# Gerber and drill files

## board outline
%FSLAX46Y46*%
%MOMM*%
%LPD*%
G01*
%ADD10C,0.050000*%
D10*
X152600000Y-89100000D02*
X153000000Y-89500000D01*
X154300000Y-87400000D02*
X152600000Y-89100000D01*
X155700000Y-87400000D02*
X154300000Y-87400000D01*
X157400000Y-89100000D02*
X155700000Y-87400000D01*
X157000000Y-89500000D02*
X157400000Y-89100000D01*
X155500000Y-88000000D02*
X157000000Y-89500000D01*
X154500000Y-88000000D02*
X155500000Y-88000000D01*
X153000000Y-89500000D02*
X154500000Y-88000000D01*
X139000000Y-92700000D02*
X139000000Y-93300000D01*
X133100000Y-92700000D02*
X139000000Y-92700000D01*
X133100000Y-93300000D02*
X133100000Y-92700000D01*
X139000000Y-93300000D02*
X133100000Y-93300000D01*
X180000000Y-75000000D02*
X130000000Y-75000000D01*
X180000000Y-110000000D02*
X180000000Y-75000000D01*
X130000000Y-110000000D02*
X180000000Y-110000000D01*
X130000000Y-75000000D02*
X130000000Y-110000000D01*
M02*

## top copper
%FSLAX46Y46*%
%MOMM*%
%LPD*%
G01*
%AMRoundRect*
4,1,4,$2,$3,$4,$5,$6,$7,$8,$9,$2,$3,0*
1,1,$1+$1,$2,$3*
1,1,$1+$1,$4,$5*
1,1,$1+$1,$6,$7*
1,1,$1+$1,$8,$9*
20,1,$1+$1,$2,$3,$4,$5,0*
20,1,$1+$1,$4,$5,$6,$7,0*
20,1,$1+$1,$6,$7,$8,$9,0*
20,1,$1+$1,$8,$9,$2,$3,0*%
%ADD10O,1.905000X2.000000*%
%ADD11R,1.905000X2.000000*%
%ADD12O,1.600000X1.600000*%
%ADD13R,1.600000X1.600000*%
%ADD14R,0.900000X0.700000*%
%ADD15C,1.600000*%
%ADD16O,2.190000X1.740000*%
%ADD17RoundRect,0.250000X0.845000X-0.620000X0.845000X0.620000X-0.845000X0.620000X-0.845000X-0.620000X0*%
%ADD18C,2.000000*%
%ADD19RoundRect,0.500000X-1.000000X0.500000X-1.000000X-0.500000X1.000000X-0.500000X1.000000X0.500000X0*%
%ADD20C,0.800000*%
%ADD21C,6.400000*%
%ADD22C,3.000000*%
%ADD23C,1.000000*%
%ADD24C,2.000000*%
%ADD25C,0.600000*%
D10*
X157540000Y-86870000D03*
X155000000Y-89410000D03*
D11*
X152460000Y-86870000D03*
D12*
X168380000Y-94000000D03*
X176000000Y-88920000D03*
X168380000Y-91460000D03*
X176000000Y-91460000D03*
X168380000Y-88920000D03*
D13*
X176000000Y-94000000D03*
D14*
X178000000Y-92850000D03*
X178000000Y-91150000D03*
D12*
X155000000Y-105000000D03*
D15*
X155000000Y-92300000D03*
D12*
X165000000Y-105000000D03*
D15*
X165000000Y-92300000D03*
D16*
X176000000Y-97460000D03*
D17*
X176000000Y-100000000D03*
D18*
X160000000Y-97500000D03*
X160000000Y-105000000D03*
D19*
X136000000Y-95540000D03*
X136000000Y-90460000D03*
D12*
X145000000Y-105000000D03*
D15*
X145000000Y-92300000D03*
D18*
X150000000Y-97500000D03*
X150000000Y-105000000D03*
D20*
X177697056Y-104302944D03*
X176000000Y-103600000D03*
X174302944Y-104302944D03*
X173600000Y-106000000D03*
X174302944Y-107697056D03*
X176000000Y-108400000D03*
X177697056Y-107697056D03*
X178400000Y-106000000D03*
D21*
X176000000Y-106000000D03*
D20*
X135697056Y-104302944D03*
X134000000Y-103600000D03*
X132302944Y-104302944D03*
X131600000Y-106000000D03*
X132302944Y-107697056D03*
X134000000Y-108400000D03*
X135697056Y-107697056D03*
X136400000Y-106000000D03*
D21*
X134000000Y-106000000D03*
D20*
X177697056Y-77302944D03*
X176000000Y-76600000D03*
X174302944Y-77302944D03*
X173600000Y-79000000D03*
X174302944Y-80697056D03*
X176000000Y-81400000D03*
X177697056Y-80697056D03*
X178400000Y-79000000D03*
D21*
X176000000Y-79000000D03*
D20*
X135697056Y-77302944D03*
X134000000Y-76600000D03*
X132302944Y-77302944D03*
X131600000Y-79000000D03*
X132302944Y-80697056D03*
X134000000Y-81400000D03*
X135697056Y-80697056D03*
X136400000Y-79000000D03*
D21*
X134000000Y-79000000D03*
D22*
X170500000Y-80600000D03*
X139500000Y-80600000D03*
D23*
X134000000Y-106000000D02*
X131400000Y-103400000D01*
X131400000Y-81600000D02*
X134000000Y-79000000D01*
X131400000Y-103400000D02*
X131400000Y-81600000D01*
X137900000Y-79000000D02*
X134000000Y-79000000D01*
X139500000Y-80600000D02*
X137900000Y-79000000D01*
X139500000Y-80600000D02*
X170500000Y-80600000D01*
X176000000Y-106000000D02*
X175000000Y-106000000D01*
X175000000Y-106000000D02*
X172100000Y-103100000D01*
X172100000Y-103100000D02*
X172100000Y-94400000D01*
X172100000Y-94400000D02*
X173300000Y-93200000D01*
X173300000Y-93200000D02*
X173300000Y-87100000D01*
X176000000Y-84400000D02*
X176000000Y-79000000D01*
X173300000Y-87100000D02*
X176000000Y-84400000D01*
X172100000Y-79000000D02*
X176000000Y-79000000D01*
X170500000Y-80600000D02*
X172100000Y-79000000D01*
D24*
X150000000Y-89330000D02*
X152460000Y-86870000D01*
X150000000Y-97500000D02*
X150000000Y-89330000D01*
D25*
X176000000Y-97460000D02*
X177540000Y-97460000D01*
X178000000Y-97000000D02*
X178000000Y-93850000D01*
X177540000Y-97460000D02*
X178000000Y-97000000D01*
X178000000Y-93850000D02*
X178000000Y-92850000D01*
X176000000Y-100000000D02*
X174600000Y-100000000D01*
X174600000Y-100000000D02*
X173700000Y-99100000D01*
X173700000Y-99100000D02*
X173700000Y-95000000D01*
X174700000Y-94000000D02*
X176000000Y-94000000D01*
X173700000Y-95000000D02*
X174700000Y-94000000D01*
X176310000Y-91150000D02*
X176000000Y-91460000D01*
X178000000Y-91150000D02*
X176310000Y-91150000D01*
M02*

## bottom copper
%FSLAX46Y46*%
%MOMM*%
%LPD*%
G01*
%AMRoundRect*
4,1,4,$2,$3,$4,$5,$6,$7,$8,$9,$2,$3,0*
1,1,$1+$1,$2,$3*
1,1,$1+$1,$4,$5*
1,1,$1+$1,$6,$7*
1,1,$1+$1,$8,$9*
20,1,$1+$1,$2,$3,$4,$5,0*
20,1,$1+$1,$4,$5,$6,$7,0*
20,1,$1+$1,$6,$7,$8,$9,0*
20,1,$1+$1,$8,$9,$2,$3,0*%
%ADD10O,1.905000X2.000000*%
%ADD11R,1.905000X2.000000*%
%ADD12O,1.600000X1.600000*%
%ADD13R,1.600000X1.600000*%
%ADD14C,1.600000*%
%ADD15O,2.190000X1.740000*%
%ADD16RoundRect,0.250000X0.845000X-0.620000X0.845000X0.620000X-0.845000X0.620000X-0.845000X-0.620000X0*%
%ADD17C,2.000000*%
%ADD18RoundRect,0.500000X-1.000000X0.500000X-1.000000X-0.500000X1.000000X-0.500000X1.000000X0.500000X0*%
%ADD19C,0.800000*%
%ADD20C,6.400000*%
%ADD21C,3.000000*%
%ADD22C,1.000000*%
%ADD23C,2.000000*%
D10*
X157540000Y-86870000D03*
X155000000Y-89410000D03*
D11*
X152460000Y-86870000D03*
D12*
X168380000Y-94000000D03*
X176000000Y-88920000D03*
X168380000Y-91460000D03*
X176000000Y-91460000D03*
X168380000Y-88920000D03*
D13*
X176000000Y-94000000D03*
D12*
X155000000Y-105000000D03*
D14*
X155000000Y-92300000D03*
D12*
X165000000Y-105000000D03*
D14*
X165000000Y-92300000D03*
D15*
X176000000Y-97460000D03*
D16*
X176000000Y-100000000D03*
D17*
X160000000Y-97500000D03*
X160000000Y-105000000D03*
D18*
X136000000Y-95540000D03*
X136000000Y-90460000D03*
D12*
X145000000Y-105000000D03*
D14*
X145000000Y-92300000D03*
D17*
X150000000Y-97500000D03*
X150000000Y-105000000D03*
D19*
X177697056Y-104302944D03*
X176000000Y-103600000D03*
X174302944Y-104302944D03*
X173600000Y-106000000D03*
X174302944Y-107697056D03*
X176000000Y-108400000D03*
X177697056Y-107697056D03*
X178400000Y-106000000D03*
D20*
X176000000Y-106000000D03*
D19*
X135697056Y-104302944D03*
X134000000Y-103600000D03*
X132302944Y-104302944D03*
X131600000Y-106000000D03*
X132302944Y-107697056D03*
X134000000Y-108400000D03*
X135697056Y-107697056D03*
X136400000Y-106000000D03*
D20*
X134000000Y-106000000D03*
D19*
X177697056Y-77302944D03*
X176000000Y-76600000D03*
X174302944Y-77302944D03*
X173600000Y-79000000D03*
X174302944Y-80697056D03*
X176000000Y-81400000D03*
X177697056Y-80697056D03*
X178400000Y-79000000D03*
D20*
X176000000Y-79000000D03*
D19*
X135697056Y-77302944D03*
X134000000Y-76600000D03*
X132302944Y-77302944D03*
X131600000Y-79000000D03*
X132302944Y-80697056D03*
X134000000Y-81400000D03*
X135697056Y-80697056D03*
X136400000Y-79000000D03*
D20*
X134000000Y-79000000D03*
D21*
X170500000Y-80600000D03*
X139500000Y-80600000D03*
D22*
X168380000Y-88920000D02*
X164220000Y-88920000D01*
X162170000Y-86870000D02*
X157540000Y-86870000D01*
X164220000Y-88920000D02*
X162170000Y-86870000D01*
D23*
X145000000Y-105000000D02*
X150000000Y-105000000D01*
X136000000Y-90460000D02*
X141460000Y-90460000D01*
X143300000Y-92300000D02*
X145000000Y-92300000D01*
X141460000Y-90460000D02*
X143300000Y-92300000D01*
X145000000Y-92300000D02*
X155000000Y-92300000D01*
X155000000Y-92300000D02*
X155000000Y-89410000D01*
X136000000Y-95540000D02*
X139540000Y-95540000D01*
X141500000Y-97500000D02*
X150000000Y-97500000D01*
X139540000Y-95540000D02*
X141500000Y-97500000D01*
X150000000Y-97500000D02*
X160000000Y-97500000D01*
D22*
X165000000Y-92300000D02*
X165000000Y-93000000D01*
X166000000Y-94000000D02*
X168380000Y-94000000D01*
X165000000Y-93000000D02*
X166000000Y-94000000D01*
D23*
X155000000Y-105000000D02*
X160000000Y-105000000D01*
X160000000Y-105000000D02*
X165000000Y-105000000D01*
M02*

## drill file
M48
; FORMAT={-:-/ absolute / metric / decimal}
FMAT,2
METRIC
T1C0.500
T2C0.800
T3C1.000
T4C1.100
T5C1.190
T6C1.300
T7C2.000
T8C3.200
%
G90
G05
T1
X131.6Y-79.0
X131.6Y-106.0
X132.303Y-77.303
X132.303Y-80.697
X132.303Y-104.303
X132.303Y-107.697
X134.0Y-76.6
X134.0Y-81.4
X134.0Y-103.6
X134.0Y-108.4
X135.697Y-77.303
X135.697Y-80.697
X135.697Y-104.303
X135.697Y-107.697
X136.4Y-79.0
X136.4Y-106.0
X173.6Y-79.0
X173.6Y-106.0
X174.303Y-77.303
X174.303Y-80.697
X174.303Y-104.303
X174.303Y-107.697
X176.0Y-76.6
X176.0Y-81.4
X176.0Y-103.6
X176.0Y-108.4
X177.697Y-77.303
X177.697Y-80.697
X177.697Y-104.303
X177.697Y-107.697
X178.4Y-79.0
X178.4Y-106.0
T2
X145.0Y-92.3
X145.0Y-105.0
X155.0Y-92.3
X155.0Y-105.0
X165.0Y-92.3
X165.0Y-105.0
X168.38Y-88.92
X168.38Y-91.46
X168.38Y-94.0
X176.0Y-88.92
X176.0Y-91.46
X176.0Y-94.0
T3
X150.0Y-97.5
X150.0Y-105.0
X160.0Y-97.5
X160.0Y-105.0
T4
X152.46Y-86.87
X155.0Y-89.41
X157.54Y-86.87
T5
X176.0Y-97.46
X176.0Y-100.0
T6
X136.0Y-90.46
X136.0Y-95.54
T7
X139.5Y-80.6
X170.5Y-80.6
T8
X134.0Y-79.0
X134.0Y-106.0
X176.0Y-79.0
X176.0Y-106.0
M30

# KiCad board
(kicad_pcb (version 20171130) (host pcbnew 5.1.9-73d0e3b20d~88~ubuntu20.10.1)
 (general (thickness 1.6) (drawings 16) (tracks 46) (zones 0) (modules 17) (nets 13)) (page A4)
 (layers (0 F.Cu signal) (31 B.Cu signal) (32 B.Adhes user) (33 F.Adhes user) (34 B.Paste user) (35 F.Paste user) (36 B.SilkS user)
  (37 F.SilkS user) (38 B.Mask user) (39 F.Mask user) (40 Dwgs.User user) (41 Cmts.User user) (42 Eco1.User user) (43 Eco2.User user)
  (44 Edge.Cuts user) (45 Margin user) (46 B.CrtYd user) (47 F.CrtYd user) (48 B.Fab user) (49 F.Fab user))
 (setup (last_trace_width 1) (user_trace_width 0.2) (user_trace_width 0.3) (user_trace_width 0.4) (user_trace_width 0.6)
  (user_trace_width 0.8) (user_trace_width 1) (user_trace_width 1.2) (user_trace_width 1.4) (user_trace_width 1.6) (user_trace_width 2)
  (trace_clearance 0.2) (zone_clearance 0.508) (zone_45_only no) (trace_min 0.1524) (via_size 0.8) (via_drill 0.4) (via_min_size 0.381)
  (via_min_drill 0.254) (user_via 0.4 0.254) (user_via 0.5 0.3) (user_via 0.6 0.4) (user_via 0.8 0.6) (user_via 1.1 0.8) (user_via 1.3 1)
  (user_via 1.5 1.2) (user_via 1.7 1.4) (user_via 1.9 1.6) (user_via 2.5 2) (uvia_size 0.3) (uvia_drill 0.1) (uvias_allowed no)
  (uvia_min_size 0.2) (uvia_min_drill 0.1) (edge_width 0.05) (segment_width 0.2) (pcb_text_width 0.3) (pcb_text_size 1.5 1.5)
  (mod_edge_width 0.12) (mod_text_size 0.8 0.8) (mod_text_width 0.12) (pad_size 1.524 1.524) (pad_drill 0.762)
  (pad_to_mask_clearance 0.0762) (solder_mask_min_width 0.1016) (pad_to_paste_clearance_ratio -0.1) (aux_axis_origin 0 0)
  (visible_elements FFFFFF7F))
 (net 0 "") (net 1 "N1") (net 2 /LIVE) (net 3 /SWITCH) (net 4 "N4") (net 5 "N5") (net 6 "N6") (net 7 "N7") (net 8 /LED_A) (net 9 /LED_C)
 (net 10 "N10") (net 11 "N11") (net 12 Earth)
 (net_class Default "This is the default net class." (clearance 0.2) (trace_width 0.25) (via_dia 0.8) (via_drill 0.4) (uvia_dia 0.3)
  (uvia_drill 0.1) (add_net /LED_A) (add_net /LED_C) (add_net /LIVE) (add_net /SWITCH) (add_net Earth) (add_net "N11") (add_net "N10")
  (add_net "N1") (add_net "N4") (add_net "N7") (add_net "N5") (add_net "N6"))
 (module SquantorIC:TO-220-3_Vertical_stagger (layer F.Cu) (at 155 85.6)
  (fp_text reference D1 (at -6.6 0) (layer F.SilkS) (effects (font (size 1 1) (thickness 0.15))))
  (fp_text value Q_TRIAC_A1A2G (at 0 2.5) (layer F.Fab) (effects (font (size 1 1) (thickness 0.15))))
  (pad 3 thru_hole oval (at 2.54 1.27) (size 1.905 2) (drill 1.1) (layers *.Cu *.Mask) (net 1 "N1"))
  (pad 2 thru_hole oval (at 0 3.81) (size 1.905 2) (drill 1.1) (layers *.Cu *.Mask) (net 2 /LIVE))
  (pad 1 thru_hole rect (at -2.54 1.27) (size 1.905 2) (drill 1.1) (layers *.Cu *.Mask) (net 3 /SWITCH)))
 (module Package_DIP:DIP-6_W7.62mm (layer F.Cu) (at 176 94 180)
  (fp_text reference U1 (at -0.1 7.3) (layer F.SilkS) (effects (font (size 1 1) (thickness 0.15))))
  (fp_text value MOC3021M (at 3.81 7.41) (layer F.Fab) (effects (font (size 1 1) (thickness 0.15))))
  (pad 6 thru_hole oval (at 7.62 0 180) (size 1.6 1.6) (drill 0.8) (layers *.Cu *.Mask) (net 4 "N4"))
  (pad 3 thru_hole oval (at 0 5.08 180) (size 1.6 1.6) (drill 0.8) (layers *.Cu *.Mask) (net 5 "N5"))
  (pad 5 thru_hole oval (at 7.62 2.54 180) (size 1.6 1.6) (drill 0.8) (layers *.Cu *.Mask) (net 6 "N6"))
  (pad 2 thru_hole oval (at 0 2.54 180) (size 1.6 1.6) (drill 0.8) (layers *.Cu *.Mask) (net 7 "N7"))
  (pad 4 thru_hole oval (at 7.62 5.08 180) (size 1.6 1.6) (drill 0.8) (layers *.Cu *.Mask) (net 1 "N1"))
  (pad 1 thru_hole rect (at 0 0 180) (size 1.6 1.6) (drill 0.8) (layers *.Cu *.Mask) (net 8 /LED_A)))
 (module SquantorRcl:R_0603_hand (layer F.Cu) (at 178 92 270)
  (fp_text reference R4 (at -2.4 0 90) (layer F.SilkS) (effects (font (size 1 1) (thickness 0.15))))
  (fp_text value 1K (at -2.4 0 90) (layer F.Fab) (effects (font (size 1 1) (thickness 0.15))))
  (pad 2 smd rect (at 0.85 0 270) (size 0.7 0.9) (layers F.Cu F.Paste F.Mask) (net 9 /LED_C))
  (pad 1 smd rect (at -0.85 0 270) (size 0.7 0.9) (layers F.Cu F.Paste F.Mask) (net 7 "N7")))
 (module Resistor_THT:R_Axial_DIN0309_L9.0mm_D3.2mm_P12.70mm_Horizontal (layer F.Cu) (at 155 92.3 270)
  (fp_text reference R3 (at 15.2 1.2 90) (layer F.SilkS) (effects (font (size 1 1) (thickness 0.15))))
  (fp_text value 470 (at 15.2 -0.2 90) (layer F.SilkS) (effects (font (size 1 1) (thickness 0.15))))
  (pad 2 thru_hole oval (at 12.7 0 270) (size 1.6 1.6) (drill 0.8) (layers *.Cu *.Mask) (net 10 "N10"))
  (pad 1 thru_hole circle (at 0 0 270) (size 1.6 1.6) (drill 0.8) (layers *.Cu *.Mask) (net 2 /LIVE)))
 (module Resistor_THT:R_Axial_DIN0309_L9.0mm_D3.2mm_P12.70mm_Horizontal (layer F.Cu) (at 165 92.3 270)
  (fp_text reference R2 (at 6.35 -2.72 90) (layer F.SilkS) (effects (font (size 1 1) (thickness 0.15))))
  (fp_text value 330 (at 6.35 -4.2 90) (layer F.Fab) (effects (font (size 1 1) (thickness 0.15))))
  (pad 2 thru_hole oval (at 12.7 0 270) (size 1.6 1.6) (drill 0.8) (layers *.Cu *.Mask) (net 10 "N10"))
  (pad 1 thru_hole circle (at 0 0 270) (size 1.6 1.6) (drill 0.8) (layers *.Cu *.Mask) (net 4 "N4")))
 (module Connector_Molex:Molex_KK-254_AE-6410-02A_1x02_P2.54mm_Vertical (layer F.Cu) (at 176 100 90)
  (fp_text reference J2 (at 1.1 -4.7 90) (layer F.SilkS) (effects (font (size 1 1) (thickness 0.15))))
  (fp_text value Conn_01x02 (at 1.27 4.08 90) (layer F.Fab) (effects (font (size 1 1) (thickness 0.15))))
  (pad 2 thru_hole oval (at 2.54 0 90) (size 1.74 2.19) (drill 1.19) (layers *.Cu *.Mask) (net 9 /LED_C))
  (pad 1 thru_hole roundrect (at 0 0 90) (size 1.74 2.19) (drill 1.19) (layers *.Cu *.Mask) (roundrect_rratio 0.143678) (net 8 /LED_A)))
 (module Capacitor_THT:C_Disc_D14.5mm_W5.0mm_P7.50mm (layer F.Cu) (at 160 105 90)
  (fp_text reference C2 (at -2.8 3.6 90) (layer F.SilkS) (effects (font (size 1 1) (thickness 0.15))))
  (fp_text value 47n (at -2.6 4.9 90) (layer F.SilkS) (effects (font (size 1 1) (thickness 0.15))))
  (pad 2 thru_hole circle (at 7.5 0 90) (size 2 2) (drill 1) (layers *.Cu *.Mask) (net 3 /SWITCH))
  (pad 1 thru_hole circle (at 0 0 90) (size 2 2) (drill 1) (layers *.Cu *.Mask) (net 10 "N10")))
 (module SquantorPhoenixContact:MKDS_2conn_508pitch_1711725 (layer F.Cu) (at 136 93 270)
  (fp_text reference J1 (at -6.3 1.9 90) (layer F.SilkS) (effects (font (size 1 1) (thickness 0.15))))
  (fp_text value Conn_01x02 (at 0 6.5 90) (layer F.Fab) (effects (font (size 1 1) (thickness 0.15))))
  (pad 2 thru_hole roundrect (at 2.54 0 270) (size 2 3) (drill 1.3) (layers *.Cu *.Mask) (roundrect_rratio 0.25) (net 3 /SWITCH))
  (pad 1 thru_hole roundrect (at -2.54 0 270) (size 2 3) (drill 1.3) (layers *.Cu *.Mask) (roundrect_rratio 0.25) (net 2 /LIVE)))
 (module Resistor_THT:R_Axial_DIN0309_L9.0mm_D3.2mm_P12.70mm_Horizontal (layer F.Cu) (at 145 92.3 270)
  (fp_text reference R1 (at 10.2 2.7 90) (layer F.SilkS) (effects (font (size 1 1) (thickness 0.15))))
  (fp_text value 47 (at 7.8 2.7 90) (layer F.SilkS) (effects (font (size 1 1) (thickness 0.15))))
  (pad 2 thru_hole oval (at 12.7 0 270) (size 1.6 1.6) (drill 0.8) (layers *.Cu *.Mask) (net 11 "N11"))
  (pad 1 thru_hole circle (at 0 0 270) (size 1.6 1.6) (drill 0.8) (layers *.Cu *.Mask) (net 2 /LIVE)))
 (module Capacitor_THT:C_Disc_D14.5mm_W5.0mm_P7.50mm (layer F.Cu) (at 150 105 90)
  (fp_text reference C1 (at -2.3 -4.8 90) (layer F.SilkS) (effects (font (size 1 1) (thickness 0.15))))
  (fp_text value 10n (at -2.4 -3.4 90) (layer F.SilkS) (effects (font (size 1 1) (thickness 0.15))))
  (pad 2 thru_hole circle (at 7.5 0 90) (size 2 2) (drill 1) (layers *.Cu *.Mask) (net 3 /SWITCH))
  (pad 1 thru_hole circle (at 0 0 90) (size 2 2) (drill 1) (layers *.Cu *.Mask) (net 11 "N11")))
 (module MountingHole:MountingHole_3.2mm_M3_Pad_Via (layer F.Cu) (at 176 106)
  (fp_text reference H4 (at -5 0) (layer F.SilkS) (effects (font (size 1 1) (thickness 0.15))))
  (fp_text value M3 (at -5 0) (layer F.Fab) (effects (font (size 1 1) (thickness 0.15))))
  (pad 1 thru_hole circle (at 1.697056 -1.697056) (size 0.8 0.8) (drill 0.5) (layers *.Cu *.Mask) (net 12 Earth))
  (pad 1 thru_hole circle (at 0 -2.4) (size 0.8 0.8) (drill 0.5) (layers *.Cu *.Mask) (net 12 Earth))
  (pad 1 thru_hole circle (at -1.697056 -1.697056) (size 0.8 0.8) (drill 0.5) (layers *.Cu *.Mask) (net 12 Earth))
  (pad 1 thru_hole circle (at -2.4 0) (size 0.8 0.8) (drill 0.5) (layers *.Cu *.Mask) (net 12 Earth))
  (pad 1 thru_hole circle (at -1.697056 1.697056) (size 0.8 0.8) (drill 0.5) (layers *.Cu *.Mask) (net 12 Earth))
  (pad 1 thru_hole circle (at 0 2.4) (size 0.8 0.8) (drill 0.5) (layers *.Cu *.Mask) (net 12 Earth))
  (pad 1 thru_hole circle (at 1.697056 1.697056) (size 0.8 0.8) (drill 0.5) (layers *.Cu *.Mask) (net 12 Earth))
  (pad 1 thru_hole circle (at 2.4 0) (size 0.8 0.8) (drill 0.5) (layers *.Cu *.Mask) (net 12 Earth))
  (pad 1 thru_hole circle (at 0 0) (size 6.4 6.4) (drill 3.2) (layers *.Cu *.Mask) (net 12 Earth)))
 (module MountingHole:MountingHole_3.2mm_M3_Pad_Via (layer F.Cu) (at 134 106)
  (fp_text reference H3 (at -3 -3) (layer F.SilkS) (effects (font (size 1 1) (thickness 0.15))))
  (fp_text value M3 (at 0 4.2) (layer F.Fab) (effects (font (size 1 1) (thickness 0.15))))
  (pad 1 thru_hole circle (at 1.697056 -1.697056) (size 0.8 0.8) (drill 0.5) (layers *.Cu *.Mask) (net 12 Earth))
  (pad 1 thru_hole circle (at 0 -2.4) (size 0.8 0.8) (drill 0.5) (layers *.Cu *.Mask) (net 12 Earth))
  (pad 1 thru_hole circle (at -1.697056 -1.697056) (size 0.8 0.8) (drill 0.5) (layers *.Cu *.Mask) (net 12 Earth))
  (pad 1 thru_hole circle (at -2.4 0) (size 0.8 0.8) (drill 0.5) (layers *.Cu *.Mask) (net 12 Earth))
  (pad 1 thru_hole circle (at -1.697056 1.697056) (size 0.8 0.8) (drill 0.5) (layers *.Cu *.Mask) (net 12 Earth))
  (pad 1 thru_hole circle (at 0 2.4) (size 0.8 0.8) (drill 0.5) (layers *.Cu *.Mask) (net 12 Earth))
  (pad 1 thru_hole circle (at 1.697056 1.697056) (size 0.8 0.8) (drill 0.5) (layers *.Cu *.Mask) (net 12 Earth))
  (pad 1 thru_hole circle (at 2.4 0) (size 0.8 0.8) (drill 0.5) (layers *.Cu *.Mask) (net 12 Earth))
  (pad 1 thru_hole circle (at 0 0) (size 6.4 6.4) (drill 3.2) (layers *.Cu *.Mask) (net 12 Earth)))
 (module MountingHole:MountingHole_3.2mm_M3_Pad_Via (layer F.Cu) (at 176 79)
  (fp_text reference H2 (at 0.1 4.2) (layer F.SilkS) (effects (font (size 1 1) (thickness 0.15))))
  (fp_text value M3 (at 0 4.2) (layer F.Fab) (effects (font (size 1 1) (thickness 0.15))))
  (pad 1 thru_hole circle (at 1.697056 -1.697056) (size 0.8 0.8) (drill 0.5) (layers *.Cu *.Mask) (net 12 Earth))
  (pad 1 thru_hole circle (at 0 -2.4) (size 0.8 0.8) (drill 0.5) (layers *.Cu *.Mask) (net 12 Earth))
  (pad 1 thru_hole circle (at -1.697056 -1.697056) (size 0.8 0.8) (drill 0.5) (layers *.Cu *.Mask) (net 12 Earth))
  (pad 1 thru_hole circle (at -2.4 0) (size 0.8 0.8) (drill 0.5) (layers *.Cu *.Mask) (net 12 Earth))
  (pad 1 thru_hole circle (at -1.697056 1.697056) (size 0.8 0.8) (drill 0.5) (layers *.Cu *.Mask) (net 12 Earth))
  (pad 1 thru_hole circle (at 0 2.4) (size 0.8 0.8) (drill 0.5) (layers *.Cu *.Mask) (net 12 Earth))
  (pad 1 thru_hole circle (at 1.697056 1.697056) (size 0.8 0.8) (drill 0.5) (layers *.Cu *.Mask) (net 12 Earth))
  (pad 1 thru_hole circle (at 2.4 0) (size 0.8 0.8) (drill 0.5) (layers *.Cu *.Mask) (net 12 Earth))
  (pad 1 thru_hole circle (at 0 0) (size 6.4 6.4) (drill 3.2) (layers *.Cu *.Mask) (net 12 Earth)))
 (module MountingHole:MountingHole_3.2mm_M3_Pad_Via (layer F.Cu) (at 134 79)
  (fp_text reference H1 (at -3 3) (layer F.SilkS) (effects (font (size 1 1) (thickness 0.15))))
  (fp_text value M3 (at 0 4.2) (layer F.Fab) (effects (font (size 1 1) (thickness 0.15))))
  (pad 1 thru_hole circle (at 1.697056 -1.697056) (size 0.8 0.8) (drill 0.5) (layers *.Cu *.Mask) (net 12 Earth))
  (pad 1 thru_hole circle (at 0 -2.4) (size 0.8 0.8) (drill 0.5) (layers *.Cu *.Mask) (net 12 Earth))
  (pad 1 thru_hole circle (at -1.697056 -1.697056) (size 0.8 0.8) (drill 0.5) (layers *.Cu *.Mask) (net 12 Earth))
  (pad 1 thru_hole circle (at -2.4 0) (size 0.8 0.8) (drill 0.5) (layers *.Cu *.Mask) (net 12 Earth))
  (pad 1 thru_hole circle (at -1.697056 1.697056) (size 0.8 0.8) (drill 0.5) (layers *.Cu *.Mask) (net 12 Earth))
  (pad 1 thru_hole circle (at 0 2.4) (size 0.8 0.8) (drill 0.5) (layers *.Cu *.Mask) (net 12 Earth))
  (pad 1 thru_hole circle (at 1.697056 1.697056) (size 0.8 0.8) (drill 0.5) (layers *.Cu *.Mask) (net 12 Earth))
  (pad 1 thru_hole circle (at 2.4 0) (size 0.8 0.8) (drill 0.5) (layers *.Cu *.Mask) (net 12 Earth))
  (pad 1 thru_hole circle (at 0 0) (size 6.4 6.4) (drill 3.2) (layers *.Cu *.Mask) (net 12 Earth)))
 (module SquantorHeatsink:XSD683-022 (layer F.Cu) (at 155 80.6)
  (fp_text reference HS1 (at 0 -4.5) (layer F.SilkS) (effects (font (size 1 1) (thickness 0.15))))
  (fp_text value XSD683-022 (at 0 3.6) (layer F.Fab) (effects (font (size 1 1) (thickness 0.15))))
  (pad 2 thru_hole circle (at 15.5 0) (size 3 3) (drill 2) (layers *.Cu *.Mask) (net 12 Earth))
  (pad 1 thru_hole circle (at -15.5 0) (size 3 3) (drill 2) (layers *.Cu *.Mask) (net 12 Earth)))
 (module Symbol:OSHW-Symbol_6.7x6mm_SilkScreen (layer B.Cu) (at 155.2 80.2 180)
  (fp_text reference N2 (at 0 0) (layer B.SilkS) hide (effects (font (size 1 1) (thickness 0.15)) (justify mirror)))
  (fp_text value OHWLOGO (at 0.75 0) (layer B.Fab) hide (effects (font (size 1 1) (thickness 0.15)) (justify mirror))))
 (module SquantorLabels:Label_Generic (layer B.Cu) (at 155.8 84.1 180)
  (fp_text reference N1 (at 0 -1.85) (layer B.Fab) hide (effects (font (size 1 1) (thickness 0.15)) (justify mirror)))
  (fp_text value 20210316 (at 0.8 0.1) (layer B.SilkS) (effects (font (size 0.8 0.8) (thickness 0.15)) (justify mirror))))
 (gr_line (start 152.6 89.1) (end 153 89.5) (layer Edge.Cuts) (width 0.05))
 (gr_line (start 154.3 87.4) (end 152.6 89.1) (layer Edge.Cuts) (width 0.05))
 (gr_line (start 155.7 87.4) (end 154.3 87.4) (layer Edge.Cuts) (width 0.05))
 (gr_line (start 157.4 89.1) (end 155.7 87.4) (layer Edge.Cuts) (width 0.05))
 (gr_line (start 157 89.5) (end 157.4 89.1) (layer Edge.Cuts) (width 0.05))
 (gr_line (start 155.5 88) (end 157 89.5) (layer Edge.Cuts) (width 0.05))
 (gr_line (start 154.5 88) (end 155.5 88) (layer Edge.Cuts) (width 0.05))
 (gr_line (start 153 89.5) (end 154.5 88) (layer Edge.Cuts) (width 0.05))
 (gr_line (start 139 92.7) (end 139 93.3) (layer Edge.Cuts) (width 0.05))
 (gr_line (start 133.1 92.7) (end 139 92.7) (layer Edge.Cuts) (width 0.05))
 (gr_line (start 133.1 93.3) (end 133.1 92.7) (layer Edge.Cuts) (width 0.05))
 (gr_line (start 139 93.3) (end 133.1 93.3) (layer Edge.Cuts) (width 0.05))
 (gr_line (start 180 75) (end 130 75) (layer Edge.Cuts) (width 0.05))
 (gr_line (start 180 110) (end 180 75) (layer Edge.Cuts) (width 0.05))
 (gr_line (start 130 110) (end 180 110) (layer Edge.Cuts) (width 0.05))
 (gr_line (start 130 75) (end 130 110) (layer Edge.Cuts) (width 0.05))
 (segment (start 168.38 88.92) (end 164.22 88.92) (width 1) (layer B.Cu) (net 1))
 (segment (start 162.17 86.87) (end 157.54 86.87) (width 1) (layer B.Cu) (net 1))
 (segment (start 164.22 88.92) (end 162.17 86.87) (width 1) (layer B.Cu) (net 1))
 (segment (start 134 106) (end 131.4 103.4) (width 1) (layer F.Cu) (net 12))
 (segment (start 131.4 81.6) (end 134 79) (width 1) (layer F.Cu) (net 12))
 (segment (start 131.4 103.4) (end 131.4 81.6) (width 1) (layer F.Cu) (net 12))
 (segment (start 137.9 79) (end 134 79) (width 1) (layer F.Cu) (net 12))
 (segment (start 139.5 80.6) (end 137.9 79) (width 1) (layer F.Cu) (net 12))
 (segment (start 139.5 80.6) (end 170.5 80.6) (width 1) (layer F.Cu) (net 12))
 (segment (start 176 106) (end 175 106) (width 1) (layer F.Cu) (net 12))
 (segment (start 175 106) (end 172.1 103.1) (width 1) (layer F.Cu) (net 12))
 (segment (start 172.1 103.1) (end 172.1 94.4) (width 1) (layer F.Cu) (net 12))
 (segment (start 172.1 94.4) (end 173.3 93.2) (width 1) (layer F.Cu) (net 12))
 (segment (start 173.3 93.2) (end 173.3 87.1) (width 1) (layer F.Cu) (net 12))
 (segment (start 176 84.4) (end 176 79) (width 1) (layer F.Cu) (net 12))
 (segment (start 173.3 87.1) (end 176 84.4) (width 1) (layer F.Cu) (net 12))
 (segment (start 172.1 79) (end 176 79) (width 1) (layer F.Cu) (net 12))
 (segment (start 170.5 80.6) (end 172.1 79) (width 1) (layer F.Cu) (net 12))
 (segment (start 145 105) (end 150 105) (width 2) (layer B.Cu) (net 11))
 (segment (start 136 90.46) (end 141.46 90.46) (width 2) (layer B.Cu) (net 2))
 (segment (start 143.3 92.3) (end 145 92.3) (width 2) (layer B.Cu) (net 2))
 (segment (start 141.46 90.46) (end 143.3 92.3) (width 2) (layer B.Cu) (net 2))
 (segment (start 145 92.3) (end 155 92.3) (width 2) (layer B.Cu) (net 2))
 (segment (start 155 92.3) (end 155 89.41) (width 2) (layer B.Cu) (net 2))
 (segment (start 136 95.54) (end 139.54 95.54) (width 2) (layer B.Cu) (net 3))
 (segment (start 141.5 97.5) (end 150 97.5) (width 2) (layer B.Cu) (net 3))
 (segment (start 139.54 95.54) (end 141.5 97.5) (width 2) (layer B.Cu) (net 3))
 (segment (start 150 97.5) (end 160 97.5) (width 2) (layer B.Cu) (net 3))
 (segment (start 150 89.33) (end 152.46 86.87) (width 2) (layer F.Cu) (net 3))
 (segment (start 150 97.5) (end 150 89.33) (width 2) (layer F.Cu) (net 3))
 (segment (start 176 97.46) (end 177.54 97.46) (width 0.6) (layer F.Cu) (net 9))
 (segment (start 178 97) (end 178 93.85) (width 0.6) (layer F.Cu) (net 9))
 (segment (start 177.54 97.46) (end 178 97) (width 0.6) (layer F.Cu) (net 9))
 (segment (start 178 93.85) (end 178 92.85) (width 0.6) (layer F.Cu) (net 9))
 (segment (start 176 100) (end 174.6 100) (width 0.6) (layer F.Cu) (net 8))
 (segment (start 174.6 100) (end 173.7 99.1) (width 0.6) (layer F.Cu) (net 8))
 (segment (start 173.7 99.1) (end 173.7 95) (width 0.6) (layer F.Cu) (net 8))
 (segment (start 174.7 94) (end 176 94) (width 0.6) (layer F.Cu) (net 8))
 (segment (start 173.7 95) (end 174.7 94) (width 0.6) (layer F.Cu) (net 8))
 (segment (start 165 92.3) (end 165 93) (width 1) (layer B.Cu) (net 4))
 (segment (start 166 94) (end 168.38 94) (width 1) (layer B.Cu) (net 4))
 (segment (start 165 93) (end 166 94) (width 1) (layer B.Cu) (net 4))
 (segment (start 176.31 91.15) (end 176 91.46) (width 0.6) (layer F.Cu) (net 7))
 (segment (start 178 91.15) (end 176.31 91.15) (width 0.6) (layer F.Cu) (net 7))
 (segment (start 155 105) (end 160 105) (width 2) (layer B.Cu) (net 10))
 (segment (start 160 105) (end 165 105) (width 2) (layer B.Cu) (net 10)))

